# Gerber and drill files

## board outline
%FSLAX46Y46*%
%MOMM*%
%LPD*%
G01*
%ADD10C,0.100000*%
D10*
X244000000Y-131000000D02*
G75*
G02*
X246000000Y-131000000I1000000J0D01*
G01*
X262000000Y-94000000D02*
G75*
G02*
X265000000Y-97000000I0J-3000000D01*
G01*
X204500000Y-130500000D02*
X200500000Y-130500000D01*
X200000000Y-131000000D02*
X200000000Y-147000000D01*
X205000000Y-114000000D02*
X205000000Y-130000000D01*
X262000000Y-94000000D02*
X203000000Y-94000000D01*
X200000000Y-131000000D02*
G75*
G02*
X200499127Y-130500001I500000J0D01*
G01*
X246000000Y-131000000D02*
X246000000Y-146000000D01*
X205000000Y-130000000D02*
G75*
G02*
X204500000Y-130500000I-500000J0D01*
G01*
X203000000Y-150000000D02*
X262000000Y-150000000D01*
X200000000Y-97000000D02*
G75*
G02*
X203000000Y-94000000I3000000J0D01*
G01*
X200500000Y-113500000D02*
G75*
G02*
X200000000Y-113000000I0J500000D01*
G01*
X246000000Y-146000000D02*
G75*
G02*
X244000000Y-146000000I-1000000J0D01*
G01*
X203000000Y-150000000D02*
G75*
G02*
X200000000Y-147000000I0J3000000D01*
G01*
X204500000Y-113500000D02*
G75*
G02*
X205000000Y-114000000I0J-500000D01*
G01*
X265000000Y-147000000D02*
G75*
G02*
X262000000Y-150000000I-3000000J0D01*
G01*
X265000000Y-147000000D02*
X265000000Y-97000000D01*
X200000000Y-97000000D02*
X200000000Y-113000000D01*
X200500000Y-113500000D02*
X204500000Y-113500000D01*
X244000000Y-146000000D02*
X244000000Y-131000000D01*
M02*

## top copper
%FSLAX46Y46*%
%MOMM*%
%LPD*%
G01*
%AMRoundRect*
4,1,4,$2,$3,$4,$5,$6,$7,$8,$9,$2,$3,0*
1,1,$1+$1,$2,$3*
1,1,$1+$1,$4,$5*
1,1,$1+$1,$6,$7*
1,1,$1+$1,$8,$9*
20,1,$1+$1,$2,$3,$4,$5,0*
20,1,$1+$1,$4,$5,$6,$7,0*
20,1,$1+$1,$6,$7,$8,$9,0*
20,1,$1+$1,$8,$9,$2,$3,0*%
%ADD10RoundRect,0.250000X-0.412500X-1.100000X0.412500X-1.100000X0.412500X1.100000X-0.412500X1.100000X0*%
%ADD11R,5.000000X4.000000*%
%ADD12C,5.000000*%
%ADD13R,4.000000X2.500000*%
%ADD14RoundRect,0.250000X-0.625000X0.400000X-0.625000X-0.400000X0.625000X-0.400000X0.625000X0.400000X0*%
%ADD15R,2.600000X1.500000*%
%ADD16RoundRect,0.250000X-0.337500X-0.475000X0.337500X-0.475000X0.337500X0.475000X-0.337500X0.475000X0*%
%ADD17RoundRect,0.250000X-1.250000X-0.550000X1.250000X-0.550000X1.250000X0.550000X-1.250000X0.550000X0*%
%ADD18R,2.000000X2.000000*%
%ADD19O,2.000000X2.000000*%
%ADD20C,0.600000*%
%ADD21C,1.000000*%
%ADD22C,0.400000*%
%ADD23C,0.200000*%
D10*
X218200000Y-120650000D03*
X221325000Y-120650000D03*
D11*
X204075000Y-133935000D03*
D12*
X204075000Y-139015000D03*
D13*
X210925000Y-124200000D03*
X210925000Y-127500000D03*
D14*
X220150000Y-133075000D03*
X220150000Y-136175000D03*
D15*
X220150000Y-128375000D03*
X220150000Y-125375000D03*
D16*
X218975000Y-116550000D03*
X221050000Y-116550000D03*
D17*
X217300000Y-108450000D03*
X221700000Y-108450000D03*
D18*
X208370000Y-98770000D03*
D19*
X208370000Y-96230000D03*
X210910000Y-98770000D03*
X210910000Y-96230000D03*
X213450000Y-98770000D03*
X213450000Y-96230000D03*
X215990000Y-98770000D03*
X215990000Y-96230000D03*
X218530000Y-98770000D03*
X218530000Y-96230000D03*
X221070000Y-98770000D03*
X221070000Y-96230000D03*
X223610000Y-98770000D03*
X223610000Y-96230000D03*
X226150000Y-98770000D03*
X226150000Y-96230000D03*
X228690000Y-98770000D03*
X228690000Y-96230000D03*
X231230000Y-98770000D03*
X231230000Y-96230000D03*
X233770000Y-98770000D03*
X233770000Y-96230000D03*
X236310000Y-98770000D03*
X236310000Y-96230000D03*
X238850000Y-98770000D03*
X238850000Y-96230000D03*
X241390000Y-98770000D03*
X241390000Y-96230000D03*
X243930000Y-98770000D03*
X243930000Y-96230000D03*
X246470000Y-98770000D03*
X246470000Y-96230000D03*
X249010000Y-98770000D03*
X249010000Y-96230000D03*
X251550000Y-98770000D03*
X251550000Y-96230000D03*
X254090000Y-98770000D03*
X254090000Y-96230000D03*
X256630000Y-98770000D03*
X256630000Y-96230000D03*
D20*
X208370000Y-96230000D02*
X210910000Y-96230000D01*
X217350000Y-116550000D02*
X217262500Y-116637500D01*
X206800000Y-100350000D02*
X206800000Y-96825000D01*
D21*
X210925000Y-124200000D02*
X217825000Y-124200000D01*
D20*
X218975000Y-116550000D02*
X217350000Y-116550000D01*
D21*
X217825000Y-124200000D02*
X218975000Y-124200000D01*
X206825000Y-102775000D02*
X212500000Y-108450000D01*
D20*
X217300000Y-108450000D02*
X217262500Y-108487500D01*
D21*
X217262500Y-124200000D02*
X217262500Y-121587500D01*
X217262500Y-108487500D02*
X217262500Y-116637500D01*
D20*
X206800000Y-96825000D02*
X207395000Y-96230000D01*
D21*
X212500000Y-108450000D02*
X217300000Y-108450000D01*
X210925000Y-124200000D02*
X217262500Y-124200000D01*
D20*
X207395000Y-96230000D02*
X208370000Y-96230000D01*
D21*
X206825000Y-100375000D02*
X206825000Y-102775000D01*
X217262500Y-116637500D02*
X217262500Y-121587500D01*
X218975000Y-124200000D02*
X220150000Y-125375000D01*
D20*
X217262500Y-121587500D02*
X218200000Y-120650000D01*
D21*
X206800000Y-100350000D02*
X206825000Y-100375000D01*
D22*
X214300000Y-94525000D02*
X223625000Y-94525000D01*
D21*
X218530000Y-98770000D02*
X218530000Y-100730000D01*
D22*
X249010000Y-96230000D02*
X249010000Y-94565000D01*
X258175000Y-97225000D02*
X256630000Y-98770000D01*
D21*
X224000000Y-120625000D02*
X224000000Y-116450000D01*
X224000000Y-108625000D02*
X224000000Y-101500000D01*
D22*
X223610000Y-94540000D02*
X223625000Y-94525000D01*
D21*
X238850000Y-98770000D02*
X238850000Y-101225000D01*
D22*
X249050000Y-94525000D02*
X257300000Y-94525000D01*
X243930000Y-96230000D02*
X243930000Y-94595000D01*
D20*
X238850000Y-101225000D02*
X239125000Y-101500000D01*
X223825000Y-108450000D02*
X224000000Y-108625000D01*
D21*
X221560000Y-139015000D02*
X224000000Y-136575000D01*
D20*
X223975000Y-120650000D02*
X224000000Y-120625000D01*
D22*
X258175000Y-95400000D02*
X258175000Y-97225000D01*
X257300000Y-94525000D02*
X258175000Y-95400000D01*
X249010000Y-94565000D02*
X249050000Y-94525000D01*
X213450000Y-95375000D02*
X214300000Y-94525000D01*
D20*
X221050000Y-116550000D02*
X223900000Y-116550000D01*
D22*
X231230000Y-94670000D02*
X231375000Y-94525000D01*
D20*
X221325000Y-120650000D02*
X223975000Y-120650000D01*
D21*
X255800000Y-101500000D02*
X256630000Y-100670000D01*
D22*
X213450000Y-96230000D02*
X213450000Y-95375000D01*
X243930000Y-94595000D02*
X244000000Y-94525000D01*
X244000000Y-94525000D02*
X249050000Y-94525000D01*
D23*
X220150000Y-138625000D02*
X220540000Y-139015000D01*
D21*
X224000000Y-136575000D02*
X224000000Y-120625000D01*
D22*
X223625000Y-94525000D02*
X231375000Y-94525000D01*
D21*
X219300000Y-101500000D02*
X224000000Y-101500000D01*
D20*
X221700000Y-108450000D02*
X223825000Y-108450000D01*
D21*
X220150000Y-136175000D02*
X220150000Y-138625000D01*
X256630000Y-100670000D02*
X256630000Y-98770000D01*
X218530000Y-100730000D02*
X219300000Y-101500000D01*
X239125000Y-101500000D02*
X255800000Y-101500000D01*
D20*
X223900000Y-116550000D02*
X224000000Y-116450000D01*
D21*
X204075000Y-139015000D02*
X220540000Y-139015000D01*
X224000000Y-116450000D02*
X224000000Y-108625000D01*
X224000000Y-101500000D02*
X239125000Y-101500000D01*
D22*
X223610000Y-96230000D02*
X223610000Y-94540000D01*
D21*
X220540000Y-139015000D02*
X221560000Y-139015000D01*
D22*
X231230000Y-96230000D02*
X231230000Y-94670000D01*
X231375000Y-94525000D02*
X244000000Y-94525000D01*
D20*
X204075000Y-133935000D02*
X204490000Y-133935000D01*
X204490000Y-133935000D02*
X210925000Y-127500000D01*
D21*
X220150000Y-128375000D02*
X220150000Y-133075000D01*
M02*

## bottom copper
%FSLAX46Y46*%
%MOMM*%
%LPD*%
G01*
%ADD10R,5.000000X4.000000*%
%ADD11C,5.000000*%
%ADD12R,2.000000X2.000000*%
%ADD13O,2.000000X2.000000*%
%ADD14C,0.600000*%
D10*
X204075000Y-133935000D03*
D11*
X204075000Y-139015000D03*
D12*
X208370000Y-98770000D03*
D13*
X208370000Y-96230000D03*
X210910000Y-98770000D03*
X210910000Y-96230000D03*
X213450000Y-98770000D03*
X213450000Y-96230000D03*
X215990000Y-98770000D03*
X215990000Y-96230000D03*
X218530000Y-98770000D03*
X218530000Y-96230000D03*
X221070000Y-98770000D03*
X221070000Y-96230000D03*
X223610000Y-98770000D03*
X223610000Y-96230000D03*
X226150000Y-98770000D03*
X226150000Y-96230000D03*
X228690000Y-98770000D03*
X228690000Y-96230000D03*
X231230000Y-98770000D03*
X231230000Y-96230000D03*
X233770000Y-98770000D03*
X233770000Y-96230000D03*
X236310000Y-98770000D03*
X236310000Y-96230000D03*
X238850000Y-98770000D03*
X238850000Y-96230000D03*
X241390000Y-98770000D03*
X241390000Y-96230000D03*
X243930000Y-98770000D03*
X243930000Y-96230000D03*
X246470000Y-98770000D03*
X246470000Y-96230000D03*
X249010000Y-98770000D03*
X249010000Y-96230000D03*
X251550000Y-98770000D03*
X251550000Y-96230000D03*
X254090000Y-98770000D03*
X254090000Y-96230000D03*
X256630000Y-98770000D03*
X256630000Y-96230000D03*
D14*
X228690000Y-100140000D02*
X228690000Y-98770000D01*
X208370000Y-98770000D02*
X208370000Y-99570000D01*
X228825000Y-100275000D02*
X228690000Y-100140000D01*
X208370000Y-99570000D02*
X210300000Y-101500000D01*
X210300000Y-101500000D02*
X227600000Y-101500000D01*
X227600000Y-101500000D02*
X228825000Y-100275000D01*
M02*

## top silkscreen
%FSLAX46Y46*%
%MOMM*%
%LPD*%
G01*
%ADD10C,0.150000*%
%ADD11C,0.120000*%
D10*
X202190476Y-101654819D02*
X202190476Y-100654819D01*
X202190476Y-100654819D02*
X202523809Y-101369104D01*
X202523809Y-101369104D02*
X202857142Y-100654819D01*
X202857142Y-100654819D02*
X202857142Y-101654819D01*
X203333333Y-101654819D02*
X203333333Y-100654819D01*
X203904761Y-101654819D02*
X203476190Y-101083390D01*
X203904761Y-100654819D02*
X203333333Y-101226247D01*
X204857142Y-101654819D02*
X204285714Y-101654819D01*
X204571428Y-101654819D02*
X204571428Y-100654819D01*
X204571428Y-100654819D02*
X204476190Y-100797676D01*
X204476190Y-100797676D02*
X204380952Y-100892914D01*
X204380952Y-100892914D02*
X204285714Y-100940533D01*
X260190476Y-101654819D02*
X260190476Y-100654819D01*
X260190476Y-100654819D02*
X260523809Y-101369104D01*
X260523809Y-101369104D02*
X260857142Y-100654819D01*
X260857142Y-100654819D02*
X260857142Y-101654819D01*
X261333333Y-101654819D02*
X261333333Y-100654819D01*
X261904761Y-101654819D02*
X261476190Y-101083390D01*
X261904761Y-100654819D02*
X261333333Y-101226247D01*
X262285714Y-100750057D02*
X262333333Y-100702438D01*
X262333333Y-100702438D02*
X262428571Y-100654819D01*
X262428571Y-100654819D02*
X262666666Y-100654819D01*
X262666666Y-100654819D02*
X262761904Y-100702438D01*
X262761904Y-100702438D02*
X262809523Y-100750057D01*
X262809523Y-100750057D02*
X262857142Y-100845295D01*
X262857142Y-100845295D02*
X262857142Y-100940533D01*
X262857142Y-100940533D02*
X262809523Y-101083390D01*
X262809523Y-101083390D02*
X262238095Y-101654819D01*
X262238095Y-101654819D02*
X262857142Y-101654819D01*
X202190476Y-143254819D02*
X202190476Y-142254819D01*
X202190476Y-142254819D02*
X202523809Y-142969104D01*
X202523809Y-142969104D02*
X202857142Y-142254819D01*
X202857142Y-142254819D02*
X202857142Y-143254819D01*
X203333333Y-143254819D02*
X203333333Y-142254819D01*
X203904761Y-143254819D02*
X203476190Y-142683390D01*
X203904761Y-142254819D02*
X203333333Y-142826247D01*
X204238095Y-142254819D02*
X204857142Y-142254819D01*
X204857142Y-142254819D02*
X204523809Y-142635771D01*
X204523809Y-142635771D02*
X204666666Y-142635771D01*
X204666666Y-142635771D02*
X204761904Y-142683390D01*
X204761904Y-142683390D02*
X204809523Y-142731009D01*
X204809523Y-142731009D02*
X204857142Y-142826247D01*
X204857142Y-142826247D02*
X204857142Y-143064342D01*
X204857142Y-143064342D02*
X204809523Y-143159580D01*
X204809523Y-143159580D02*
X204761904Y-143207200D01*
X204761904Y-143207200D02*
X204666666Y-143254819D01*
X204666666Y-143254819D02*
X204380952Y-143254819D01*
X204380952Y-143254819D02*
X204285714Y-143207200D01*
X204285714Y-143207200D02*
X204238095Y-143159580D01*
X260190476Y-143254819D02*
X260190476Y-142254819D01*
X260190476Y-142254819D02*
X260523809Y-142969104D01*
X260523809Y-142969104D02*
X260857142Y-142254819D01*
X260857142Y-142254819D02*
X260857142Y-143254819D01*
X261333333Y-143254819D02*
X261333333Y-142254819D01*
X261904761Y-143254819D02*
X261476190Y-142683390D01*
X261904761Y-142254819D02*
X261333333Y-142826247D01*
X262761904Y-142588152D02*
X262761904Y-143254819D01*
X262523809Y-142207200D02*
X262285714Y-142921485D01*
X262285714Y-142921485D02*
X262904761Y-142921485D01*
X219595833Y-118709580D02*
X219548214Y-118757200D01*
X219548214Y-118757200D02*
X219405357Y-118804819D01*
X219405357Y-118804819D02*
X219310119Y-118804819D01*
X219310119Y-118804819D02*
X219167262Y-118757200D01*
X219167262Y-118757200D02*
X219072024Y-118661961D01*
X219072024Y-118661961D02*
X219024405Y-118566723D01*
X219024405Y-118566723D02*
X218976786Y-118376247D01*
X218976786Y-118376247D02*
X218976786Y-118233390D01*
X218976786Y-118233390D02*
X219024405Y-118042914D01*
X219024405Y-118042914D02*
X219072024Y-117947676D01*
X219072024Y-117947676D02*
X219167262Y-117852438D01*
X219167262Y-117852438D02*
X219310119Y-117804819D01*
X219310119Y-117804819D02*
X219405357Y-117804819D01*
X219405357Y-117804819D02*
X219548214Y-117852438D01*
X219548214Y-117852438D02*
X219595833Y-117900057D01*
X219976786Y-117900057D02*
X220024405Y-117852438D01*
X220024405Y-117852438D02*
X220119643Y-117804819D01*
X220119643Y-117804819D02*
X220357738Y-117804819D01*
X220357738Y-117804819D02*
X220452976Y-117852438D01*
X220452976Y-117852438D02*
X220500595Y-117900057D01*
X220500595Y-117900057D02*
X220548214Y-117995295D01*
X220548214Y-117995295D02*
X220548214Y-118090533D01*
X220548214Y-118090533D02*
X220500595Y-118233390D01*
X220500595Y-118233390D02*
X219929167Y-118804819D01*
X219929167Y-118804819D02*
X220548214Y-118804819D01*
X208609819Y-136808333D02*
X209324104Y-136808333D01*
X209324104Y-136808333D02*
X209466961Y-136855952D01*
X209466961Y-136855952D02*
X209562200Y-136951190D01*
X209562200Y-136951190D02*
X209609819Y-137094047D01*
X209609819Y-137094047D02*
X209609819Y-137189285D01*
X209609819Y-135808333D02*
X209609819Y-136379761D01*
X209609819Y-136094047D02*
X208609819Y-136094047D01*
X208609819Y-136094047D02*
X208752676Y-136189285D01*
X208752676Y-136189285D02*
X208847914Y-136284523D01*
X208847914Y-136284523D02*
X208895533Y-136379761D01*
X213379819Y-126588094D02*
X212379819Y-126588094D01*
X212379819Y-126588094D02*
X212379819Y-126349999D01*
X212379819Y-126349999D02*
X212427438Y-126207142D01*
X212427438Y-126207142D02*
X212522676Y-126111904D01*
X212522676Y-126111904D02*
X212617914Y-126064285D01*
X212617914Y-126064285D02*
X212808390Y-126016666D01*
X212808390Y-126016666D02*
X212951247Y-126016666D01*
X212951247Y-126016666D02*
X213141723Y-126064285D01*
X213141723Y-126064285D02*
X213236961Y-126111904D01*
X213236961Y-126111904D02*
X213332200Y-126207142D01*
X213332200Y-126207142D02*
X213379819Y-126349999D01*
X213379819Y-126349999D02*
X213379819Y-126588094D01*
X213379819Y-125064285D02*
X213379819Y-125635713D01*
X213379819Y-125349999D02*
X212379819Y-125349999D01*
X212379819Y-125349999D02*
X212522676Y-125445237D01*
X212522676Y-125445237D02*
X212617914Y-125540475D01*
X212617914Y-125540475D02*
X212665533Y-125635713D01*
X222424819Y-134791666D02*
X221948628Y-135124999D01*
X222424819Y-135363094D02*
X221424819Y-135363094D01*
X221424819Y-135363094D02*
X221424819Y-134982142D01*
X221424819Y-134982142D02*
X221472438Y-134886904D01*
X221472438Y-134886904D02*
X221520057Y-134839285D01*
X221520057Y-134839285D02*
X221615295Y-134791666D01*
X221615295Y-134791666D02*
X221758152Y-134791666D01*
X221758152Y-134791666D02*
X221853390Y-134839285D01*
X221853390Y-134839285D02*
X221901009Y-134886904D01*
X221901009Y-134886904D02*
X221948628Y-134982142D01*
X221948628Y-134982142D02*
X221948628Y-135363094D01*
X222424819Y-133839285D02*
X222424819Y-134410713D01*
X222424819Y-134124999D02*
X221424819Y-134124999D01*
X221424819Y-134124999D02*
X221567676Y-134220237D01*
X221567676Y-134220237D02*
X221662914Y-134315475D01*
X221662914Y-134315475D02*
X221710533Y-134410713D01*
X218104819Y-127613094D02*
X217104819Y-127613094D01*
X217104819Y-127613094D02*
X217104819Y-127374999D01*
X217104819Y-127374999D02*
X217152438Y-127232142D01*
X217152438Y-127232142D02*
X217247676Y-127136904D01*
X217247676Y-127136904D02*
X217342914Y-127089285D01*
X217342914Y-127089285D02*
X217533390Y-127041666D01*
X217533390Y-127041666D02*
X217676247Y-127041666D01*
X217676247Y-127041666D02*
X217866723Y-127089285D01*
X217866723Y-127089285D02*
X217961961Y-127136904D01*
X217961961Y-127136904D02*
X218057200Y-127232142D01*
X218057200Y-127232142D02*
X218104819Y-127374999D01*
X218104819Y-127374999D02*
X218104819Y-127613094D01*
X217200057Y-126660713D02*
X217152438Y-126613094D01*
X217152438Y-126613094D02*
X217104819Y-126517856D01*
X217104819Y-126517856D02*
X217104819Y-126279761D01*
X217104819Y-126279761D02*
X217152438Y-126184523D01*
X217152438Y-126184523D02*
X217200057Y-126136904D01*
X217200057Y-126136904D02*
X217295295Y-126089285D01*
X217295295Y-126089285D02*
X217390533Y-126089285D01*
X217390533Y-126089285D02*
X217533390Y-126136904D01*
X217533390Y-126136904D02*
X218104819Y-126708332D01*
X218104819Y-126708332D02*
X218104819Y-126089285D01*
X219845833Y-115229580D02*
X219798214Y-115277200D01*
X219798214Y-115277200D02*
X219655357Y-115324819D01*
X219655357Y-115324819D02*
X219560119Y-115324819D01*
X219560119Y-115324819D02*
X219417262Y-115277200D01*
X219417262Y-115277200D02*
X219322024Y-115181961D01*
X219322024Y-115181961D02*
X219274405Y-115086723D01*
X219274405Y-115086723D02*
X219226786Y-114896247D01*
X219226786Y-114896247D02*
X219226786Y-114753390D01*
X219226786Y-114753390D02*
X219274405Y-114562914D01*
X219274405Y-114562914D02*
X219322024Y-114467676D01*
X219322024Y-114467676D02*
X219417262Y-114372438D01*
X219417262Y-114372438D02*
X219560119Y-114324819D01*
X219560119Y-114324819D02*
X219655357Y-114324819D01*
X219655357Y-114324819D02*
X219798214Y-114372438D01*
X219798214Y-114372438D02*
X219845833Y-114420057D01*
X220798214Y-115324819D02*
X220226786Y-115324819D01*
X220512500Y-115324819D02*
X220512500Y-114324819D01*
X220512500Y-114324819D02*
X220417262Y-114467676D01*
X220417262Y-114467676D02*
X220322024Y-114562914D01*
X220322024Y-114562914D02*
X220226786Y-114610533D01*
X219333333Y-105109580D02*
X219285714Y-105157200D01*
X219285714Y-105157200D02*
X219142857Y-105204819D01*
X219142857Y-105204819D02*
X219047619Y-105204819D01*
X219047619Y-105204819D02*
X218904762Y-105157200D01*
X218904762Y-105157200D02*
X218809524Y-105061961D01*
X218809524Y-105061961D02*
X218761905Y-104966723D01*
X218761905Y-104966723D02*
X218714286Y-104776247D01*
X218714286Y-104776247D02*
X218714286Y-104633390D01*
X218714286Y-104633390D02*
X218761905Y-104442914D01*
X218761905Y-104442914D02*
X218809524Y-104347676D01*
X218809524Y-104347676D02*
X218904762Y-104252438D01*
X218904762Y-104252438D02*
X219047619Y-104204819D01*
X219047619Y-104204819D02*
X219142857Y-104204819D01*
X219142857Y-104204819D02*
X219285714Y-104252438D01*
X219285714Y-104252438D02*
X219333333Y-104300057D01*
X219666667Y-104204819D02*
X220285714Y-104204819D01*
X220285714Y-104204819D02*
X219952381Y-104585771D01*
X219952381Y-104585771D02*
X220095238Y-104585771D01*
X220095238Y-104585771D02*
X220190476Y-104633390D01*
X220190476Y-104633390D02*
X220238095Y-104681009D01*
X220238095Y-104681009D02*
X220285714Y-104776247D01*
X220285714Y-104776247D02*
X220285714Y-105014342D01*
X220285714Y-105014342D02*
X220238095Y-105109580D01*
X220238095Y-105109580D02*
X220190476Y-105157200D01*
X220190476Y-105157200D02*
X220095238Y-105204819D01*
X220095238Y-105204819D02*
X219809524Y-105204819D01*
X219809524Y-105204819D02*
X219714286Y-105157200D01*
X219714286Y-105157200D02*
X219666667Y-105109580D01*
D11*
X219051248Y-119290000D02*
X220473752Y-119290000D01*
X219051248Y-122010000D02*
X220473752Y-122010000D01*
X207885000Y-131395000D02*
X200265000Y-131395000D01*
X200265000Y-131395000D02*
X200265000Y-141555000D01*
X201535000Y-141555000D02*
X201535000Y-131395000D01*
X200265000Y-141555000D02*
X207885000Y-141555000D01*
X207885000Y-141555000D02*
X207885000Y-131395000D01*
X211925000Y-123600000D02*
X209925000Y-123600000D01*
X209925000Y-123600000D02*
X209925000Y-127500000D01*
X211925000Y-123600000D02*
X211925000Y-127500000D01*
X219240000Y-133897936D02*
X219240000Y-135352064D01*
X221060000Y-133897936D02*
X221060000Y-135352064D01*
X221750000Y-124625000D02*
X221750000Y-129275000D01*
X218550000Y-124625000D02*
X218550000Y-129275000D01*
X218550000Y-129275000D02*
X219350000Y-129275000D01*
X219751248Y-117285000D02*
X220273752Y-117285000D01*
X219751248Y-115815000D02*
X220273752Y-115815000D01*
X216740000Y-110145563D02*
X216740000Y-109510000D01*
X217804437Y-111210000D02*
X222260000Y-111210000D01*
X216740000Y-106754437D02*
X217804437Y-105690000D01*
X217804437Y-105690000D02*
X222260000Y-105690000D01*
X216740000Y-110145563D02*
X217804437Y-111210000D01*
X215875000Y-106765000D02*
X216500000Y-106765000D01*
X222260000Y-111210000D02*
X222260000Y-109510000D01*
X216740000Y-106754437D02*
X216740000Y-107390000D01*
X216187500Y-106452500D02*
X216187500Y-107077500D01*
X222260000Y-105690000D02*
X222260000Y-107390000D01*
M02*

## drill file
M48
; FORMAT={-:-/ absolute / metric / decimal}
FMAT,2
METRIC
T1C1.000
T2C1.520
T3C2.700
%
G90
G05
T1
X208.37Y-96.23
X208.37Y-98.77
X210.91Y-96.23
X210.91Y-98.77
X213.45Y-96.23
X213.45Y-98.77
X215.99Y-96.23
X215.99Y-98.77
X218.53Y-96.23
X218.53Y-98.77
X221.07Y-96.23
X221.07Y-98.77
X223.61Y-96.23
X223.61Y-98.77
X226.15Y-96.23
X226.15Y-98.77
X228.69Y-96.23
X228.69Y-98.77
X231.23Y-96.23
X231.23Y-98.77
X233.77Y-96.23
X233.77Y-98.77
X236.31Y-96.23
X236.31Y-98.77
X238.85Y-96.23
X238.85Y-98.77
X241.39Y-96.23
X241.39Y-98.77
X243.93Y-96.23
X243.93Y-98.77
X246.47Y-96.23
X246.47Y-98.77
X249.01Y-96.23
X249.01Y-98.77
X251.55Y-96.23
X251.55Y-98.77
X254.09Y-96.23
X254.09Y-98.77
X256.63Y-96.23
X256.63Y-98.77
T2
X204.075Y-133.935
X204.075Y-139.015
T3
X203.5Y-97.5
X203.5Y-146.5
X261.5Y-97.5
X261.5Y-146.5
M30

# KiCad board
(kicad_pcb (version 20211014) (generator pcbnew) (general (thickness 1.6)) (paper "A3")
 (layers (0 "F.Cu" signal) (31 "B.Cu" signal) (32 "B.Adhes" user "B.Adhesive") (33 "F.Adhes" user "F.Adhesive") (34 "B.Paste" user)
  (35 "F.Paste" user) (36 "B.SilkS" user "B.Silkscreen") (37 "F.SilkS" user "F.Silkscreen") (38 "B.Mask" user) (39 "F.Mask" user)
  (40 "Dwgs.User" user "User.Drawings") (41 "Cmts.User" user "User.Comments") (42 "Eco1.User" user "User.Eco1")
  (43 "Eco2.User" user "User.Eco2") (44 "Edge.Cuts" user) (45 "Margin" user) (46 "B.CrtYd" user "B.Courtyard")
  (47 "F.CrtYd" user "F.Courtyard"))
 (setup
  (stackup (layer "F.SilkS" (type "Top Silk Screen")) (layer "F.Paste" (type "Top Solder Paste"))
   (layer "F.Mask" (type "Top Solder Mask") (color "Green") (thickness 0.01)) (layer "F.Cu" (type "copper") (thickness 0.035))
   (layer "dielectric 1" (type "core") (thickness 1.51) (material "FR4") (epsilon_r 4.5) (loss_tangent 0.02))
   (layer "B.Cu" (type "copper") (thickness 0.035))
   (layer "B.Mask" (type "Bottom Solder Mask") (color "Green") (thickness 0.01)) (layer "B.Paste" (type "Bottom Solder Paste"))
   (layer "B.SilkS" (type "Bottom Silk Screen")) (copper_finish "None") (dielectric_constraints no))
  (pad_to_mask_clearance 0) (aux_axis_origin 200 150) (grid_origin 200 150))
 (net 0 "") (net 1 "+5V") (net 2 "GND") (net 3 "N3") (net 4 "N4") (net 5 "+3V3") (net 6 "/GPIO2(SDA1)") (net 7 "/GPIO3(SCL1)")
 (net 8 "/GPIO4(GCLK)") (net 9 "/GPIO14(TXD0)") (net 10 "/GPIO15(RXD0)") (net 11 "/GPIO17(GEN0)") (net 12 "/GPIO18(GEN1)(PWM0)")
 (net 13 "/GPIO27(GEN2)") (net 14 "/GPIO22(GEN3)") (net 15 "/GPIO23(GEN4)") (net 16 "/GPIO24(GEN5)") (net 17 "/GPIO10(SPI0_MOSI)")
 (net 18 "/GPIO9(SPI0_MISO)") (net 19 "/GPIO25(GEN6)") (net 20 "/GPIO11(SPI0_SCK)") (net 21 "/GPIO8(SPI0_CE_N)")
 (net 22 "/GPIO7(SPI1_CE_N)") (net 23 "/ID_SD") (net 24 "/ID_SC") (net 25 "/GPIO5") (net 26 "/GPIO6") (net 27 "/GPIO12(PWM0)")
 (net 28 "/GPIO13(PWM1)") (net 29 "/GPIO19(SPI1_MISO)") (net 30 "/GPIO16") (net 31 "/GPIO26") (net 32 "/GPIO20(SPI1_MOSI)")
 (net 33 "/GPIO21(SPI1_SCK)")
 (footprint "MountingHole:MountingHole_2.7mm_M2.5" (layer "F.Cu") (at 203.5 97.5 180)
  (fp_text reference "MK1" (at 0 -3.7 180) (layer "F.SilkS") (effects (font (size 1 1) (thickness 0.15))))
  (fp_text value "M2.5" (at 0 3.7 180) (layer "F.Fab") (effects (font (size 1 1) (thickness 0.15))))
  (pad "" np_thru_hole circle locked (at 0 0 180) (size 2.7 2.7) (drill 2.7) (layers *.Cu *.Mask)))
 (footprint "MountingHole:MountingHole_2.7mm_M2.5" (layer "F.Cu") (at 261.5 97.5 180)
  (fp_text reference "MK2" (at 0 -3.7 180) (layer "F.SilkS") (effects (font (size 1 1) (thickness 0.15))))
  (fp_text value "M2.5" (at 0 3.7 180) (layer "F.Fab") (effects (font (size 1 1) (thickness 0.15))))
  (pad "" np_thru_hole circle locked (at 0 0 180) (size 2.7 2.7) (drill 2.7) (layers *.Cu *.Mask)))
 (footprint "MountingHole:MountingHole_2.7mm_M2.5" (layer "F.Cu") (at 203.5 146.5)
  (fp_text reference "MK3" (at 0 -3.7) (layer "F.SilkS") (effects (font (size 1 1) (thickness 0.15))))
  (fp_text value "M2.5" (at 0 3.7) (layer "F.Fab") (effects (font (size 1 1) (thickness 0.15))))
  (pad "" np_thru_hole circle locked (at 0 0) (size 2.7 2.7) (drill 2.7) (layers *.Cu *.Mask)))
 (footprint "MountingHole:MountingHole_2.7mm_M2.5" (layer "F.Cu") (at 261.5 146.5)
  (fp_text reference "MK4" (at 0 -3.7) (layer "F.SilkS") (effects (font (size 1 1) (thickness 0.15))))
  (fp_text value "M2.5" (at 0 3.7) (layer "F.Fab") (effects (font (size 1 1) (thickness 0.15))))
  (pad "" np_thru_hole circle locked (at 0 0) (size 2.7 2.7) (drill 2.7) (layers *.Cu *.Mask)))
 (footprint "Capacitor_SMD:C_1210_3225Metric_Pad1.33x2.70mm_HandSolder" (layer "F.Cu") (at 219.7625 120.65)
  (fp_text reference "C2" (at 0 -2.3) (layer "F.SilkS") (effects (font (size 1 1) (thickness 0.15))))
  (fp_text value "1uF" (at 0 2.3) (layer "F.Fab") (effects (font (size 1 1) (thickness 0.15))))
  (fp_line (start -0.711252 -1.36) (end 0.711252 -1.36) (layer "F.SilkS") (width 0.12))
  (fp_line (start -0.711252 1.36) (end 0.711252 1.36) (layer "F.SilkS") (width 0.12))
  (pad "1" smd roundrect locked (at -1.5625 0) (size 1.325 2.7) (layers "F.Cu" "F.Paste" "F.Mask") (roundrect_rratio 0.1886792453)
   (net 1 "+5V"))
  (pad "2" smd roundrect locked (at 1.5625 0) (size 1.325 2.7) (layers "F.Cu" "F.Paste" "F.Mask") (roundrect_rratio 0.1886792453)
   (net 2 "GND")))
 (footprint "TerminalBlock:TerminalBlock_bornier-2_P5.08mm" (layer "F.Cu") (at 204.075 133.935 -90)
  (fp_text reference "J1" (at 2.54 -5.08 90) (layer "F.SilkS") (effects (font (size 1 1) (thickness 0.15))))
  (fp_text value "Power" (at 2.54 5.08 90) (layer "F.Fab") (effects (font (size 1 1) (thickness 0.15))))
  (fp_line (start -2.54 -3.81) (end -2.54 3.81) (layer "F.SilkS") (width 0.12))
  (fp_line (start -2.54 3.81) (end 7.62 3.81) (layer "F.SilkS") (width 0.12))
  (fp_line (start 7.62 2.54) (end -2.54 2.54) (layer "F.SilkS") (width 0.12))
  (fp_line (start 7.62 3.81) (end 7.62 -3.81) (layer "F.SilkS") (width 0.12))
  (fp_line (start 7.62 -3.81) (end -2.54 -3.81) (layer "F.SilkS") (width 0.12))
  (pad "1" thru_hole rect locked (at 0 0 270) (size 4 5) (drill 1.52) (layers *.Cu *.Mask) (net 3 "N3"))
  (pad "2" thru_hole circle locked (at 5.08 0 270) (size 5 5) (drill 1.52) (layers *.Cu *.Mask) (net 2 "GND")))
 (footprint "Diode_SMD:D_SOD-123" (layer "F.Cu") (at 210.925 125.85 -90)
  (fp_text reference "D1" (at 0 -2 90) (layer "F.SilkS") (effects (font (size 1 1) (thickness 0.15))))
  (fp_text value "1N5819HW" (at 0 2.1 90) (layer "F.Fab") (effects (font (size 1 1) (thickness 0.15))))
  (fp_line (start -2.25 -1) (end -2.25 1) (layer "F.SilkS") (width 0.12))
  (fp_line (start -2.25 1) (end 1.65 1) (layer "F.SilkS") (width 0.12))
  (fp_line (start -2.25 -1) (end 1.65 -1) (layer "F.SilkS") (width 0.12))
  (pad "1" smd rect locked (at -1.65 0 270) (size 2.5 4) (layers "F.Cu" "F.Paste" "F.Mask") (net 1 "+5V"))
  (pad "2" smd rect locked (at 1.65 0 270) (size 2.5 4) (layers "F.Cu" "F.Paste" "F.Mask") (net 3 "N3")))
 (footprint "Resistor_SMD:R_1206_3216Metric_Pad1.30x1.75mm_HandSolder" (layer "F.Cu") (at 220.15 134.625 -90)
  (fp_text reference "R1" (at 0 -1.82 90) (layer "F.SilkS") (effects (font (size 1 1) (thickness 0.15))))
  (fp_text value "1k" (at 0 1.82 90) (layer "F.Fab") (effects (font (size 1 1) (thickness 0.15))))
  (fp_line (start -0.727064 0.91) (end 0.727064 0.91) (layer "F.SilkS") (width 0.12))
  (fp_line (start -0.727064 -0.91) (end 0.727064 -0.91) (layer "F.SilkS") (width 0.12))
  (pad "1" smd roundrect locked (at -1.55 0 270) (size 1.3 1.75) (layers "F.Cu" "F.Paste" "F.Mask") (roundrect_rratio 0.1923076923)
   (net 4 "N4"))
  (pad "2" smd roundrect locked (at 1.55 0 270) (size 1.3 1.75) (layers "F.Cu" "F.Paste" "F.Mask") (roundrect_rratio 0.1923076923)
   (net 2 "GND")))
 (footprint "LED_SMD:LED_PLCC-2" (layer "F.Cu") (at 220.15 126.875 90)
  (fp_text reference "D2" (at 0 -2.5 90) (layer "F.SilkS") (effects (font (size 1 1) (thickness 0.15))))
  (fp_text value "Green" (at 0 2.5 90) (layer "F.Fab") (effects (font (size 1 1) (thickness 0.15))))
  (fp_line (start 2.25 1.6) (end -2.4 1.6) (layer "F.SilkS") (width 0.12))
  (fp_line (start 2.25 -1.6) (end -2.4 -1.6) (layer "F.SilkS") (width 0.12))
  (fp_line (start -2.4 -1.6) (end -2.4 -0.8) (layer "F.SilkS") (width 0.12))
  (pad "1" smd rect locked (at -1.5 0 90) (size 1.5 2.6) (layers "F.Cu" "F.Paste" "F.Mask") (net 4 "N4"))
  (pad "2" smd rect locked (at 1.5 0 90) (size 1.5 2.6) (layers "F.Cu" "F.Paste" "F.Mask") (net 1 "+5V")))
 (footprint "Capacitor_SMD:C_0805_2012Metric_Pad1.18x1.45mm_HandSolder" (layer "F.Cu") (at 220.0125 116.55)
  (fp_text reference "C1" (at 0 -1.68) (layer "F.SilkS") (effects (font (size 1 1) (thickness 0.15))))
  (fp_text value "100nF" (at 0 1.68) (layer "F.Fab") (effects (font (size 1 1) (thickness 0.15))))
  (fp_line (start -0.261252 0.735) (end 0.261252 0.735) (layer "F.SilkS") (width 0.12))
  (fp_line (start -0.261252 -0.735) (end 0.261252 -0.735) (layer "F.SilkS") (width 0.12))
  (pad "1" smd roundrect locked (at -1.0375 0) (size 1.175 1.45) (layers "F.Cu" "F.Paste" "F.Mask") (roundrect_rratio 0.2127659574)
   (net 1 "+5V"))
  (pad "2" smd roundrect locked (at 1.0375 0) (size 1.175 1.45) (layers "F.Cu" "F.Paste" "F.Mask") (roundrect_rratio 0.2127659574)
   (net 2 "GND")))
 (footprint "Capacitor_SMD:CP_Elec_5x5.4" (layer "F.Cu") (at 219.5 108.45)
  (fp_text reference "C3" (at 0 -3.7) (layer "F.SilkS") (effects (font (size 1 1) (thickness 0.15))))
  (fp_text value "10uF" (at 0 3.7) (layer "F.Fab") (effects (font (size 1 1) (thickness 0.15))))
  (fp_line (start -2.76 1.695563) (end -2.76 1.06) (layer "F.SilkS") (width 0.12))
  (fp_line (start -1.695563 2.76) (end 2.76 2.76) (layer "F.SilkS") (width 0.12))
  (fp_line (start -2.76 -1.695563) (end -1.695563 -2.76) (layer "F.SilkS") (width 0.12))
  (fp_line (start -1.695563 -2.76) (end 2.76 -2.76) (layer "F.SilkS") (width 0.12))
  (fp_line (start -2.76 1.695563) (end -1.695563 2.76) (layer "F.SilkS") (width 0.12))
  (fp_line (start -3.625 -1.685) (end -3 -1.685) (layer "F.SilkS") (width 0.12))
  (fp_line (start 2.76 2.76) (end 2.76 1.06) (layer "F.SilkS") (width 0.12))
  (fp_line (start -2.76 -1.695563) (end -2.76 -1.06) (layer "F.SilkS") (width 0.12))
  (fp_line (start -3.3125 -1.9975) (end -3.3125 -1.3725) (layer "F.SilkS") (width 0.12))
  (fp_line (start 2.76 -2.76) (end 2.76 -1.06) (layer "F.SilkS") (width 0.12))
  (pad "1" smd roundrect locked (at -2.2 0) (size 3 1.6) (layers "F.Cu" "F.Paste" "F.Mask") (roundrect_rratio 0.15625) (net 1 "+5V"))
  (pad "2" smd roundrect locked (at 2.2 0) (size 3 1.6) (layers "F.Cu" "F.Paste" "F.Mask") (roundrect_rratio 0.15625) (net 2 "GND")))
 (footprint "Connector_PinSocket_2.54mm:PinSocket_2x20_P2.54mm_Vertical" (layer "B.Cu") (at 208.37 98.77 -90)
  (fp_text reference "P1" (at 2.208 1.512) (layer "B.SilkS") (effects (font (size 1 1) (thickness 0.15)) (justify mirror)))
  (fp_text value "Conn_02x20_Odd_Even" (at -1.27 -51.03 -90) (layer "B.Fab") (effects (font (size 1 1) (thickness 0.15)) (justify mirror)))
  (pad "1" thru_hole rect locked (at 0 0 270) (size 2 2) (drill 1) (layers *.Cu *.Mask) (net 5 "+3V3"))
  (pad "2" thru_hole oval locked (at -2.54 0 270) (size 2 2) (drill 1) (layers *.Cu *.Mask) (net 1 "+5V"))
  (pad "3" thru_hole oval locked (at 0 -2.54 270) (size 2 2) (drill 1) (layers *.Cu *.Mask) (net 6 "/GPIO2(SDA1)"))
  (pad "4" thru_hole oval locked (at -2.54 -2.54 270) (size 2 2) (drill 1) (layers *.Cu *.Mask) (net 1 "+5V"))
  (pad "5" thru_hole oval locked (at 0 -5.08 270) (size 2 2) (drill 1) (layers *.Cu *.Mask) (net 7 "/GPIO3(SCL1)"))
  (pad "6" thru_hole oval locked (at -2.54 -5.08 270) (size 2 2) (drill 1) (layers *.Cu *.Mask) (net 2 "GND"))
  (pad "7" thru_hole oval locked (at 0 -7.62 270) (size 2 2) (drill 1) (layers *.Cu *.Mask) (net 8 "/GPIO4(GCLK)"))
  (pad "8" thru_hole oval locked (at -2.54 -7.62 270) (size 2 2) (drill 1) (layers *.Cu *.Mask) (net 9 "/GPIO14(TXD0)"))
  (pad "9" thru_hole oval locked (at 0 -10.16 270) (size 2 2) (drill 1) (layers *.Cu *.Mask) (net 2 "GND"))
  (pad "10" thru_hole oval locked (at -2.54 -10.16 270) (size 2 2) (drill 1) (layers *.Cu *.Mask) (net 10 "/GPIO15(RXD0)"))
  (pad "11" thru_hole oval locked (at 0 -12.7 270) (size 2 2) (drill 1) (layers *.Cu *.Mask) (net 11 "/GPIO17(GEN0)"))
  (pad "12" thru_hole oval locked (at -2.54 -12.7 270) (size 2 2) (drill 1) (layers *.Cu *.Mask) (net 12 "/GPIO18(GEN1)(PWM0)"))
  (pad "13" thru_hole oval locked (at 0 -15.24 270) (size 2 2) (drill 1) (layers *.Cu *.Mask) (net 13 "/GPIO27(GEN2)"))
  (pad "14" thru_hole oval locked (at -2.54 -15.24 270) (size 2 2) (drill 1) (layers *.Cu *.Mask) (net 2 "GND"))
  (pad "15" thru_hole oval locked (at 0 -17.78 270) (size 2 2) (drill 1) (layers *.Cu *.Mask) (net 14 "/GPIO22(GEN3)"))
  (pad "16" thru_hole oval locked (at -2.54 -17.78 270) (size 2 2) (drill 1) (layers *.Cu *.Mask) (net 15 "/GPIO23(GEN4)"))
  (pad "17" thru_hole oval locked (at 0 -20.32 270) (size 2 2) (drill 1) (layers *.Cu *.Mask) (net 5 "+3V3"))
  (pad "18" thru_hole oval locked (at -2.54 -20.32 270) (size 2 2) (drill 1) (layers *.Cu *.Mask) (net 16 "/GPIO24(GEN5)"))
  (pad "19" thru_hole oval locked (at 0 -22.86 270) (size 2 2) (drill 1) (layers *.Cu *.Mask) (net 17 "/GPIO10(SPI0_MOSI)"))
  (pad "20" thru_hole oval locked (at -2.54 -22.86 270) (size 2 2) (drill 1) (layers *.Cu *.Mask) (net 2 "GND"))
  (pad "21" thru_hole oval locked (at 0 -25.4 270) (size 2 2) (drill 1) (layers *.Cu *.Mask) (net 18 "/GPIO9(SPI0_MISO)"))
  (pad "22" thru_hole oval locked (at -2.54 -25.4 270) (size 2 2) (drill 1) (layers *.Cu *.Mask) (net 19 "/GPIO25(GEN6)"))
  (pad "23" thru_hole oval locked (at 0 -27.94 270) (size 2 2) (drill 1) (layers *.Cu *.Mask) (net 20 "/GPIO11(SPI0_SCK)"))
  (pad "24" thru_hole oval locked (at -2.54 -27.94 270) (size 2 2) (drill 1) (layers *.Cu *.Mask) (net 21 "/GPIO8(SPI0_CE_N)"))
  (pad "25" thru_hole oval locked (at 0 -30.48 270) (size 2 2) (drill 1) (layers *.Cu *.Mask) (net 2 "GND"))
  (pad "26" thru_hole oval locked (at -2.54 -30.48 270) (size 2 2) (drill 1) (layers *.Cu *.Mask) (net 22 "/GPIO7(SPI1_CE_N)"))
  (pad "27" thru_hole oval locked (at 0 -33.02 270) (size 2 2) (drill 1) (layers *.Cu *.Mask) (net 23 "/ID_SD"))
  (pad "28" thru_hole oval locked (at -2.54 -33.02 270) (size 2 2) (drill 1) (layers *.Cu *.Mask) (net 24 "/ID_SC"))
  (pad "29" thru_hole oval locked (at 0 -35.56 270) (size 2 2) (drill 1) (layers *.Cu *.Mask) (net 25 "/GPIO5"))
  (pad "30" thru_hole oval locked (at -2.54 -35.56 270) (size 2 2) (drill 1) (layers *.Cu *.Mask) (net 2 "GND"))
  (pad "31" thru_hole oval locked (at 0 -38.1 270) (size 2 2) (drill 1) (layers *.Cu *.Mask) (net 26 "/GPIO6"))
  (pad "32" thru_hole oval locked (at -2.54 -38.1 270) (size 2 2) (drill 1) (layers *.Cu *.Mask) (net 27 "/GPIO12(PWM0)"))
  (pad "33" thru_hole oval locked (at 0 -40.64 270) (size 2 2) (drill 1) (layers *.Cu *.Mask) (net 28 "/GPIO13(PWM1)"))
  (pad "34" thru_hole oval locked (at -2.54 -40.64 270) (size 2 2) (drill 1) (layers *.Cu *.Mask) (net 2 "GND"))
  (pad "35" thru_hole oval locked (at 0 -43.18 270) (size 2 2) (drill 1) (layers *.Cu *.Mask) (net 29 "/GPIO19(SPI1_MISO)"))
  (pad "36" thru_hole oval locked (at -2.54 -43.18 270) (size 2 2) (drill 1) (layers *.Cu *.Mask) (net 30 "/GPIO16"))
  (pad "37" thru_hole oval locked (at 0 -45.72 270) (size 2 2) (drill 1) (layers *.Cu *.Mask) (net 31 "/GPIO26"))
  (pad "38" thru_hole oval locked (at -2.54 -45.72 270) (size 2 2) (drill 1) (layers *.Cu *.Mask) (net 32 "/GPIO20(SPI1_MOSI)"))
  (pad "39" thru_hole oval locked (at 0 -48.26 270) (size 2 2) (drill 1) (layers *.Cu *.Mask) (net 2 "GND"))
  (pad "40" thru_hole oval locked (at -2.54 -48.26 270) (size 2 2) (drill 1) (layers *.Cu *.Mask) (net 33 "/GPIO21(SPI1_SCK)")))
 (gr_arc (start 244 131) (mid 245 130) (end 246 131) (layer "Edge.Cuts") (width 0.1))
 (gr_arc (start 262 94) (mid 264.12132 94.87868) (end 265 97) (layer "Edge.Cuts") (width 0.1))
 (gr_line (start 204.5 130.5) (end 200.5 130.5) (layer "Edge.Cuts") (width 0.1))
 (gr_line (start 200 131) (end 200 147) (layer "Edge.Cuts") (width 0.1))
 (gr_line (start 205 114) (end 205 130) (layer "Edge.Cuts") (width 0.1))
 (gr_line (start 262 94) (end 203 94) (layer "Edge.Cuts") (width 0.1))
 (gr_arc (start 200 131) (mid 200.146138 130.646755) (end 200.499127 130.500001) (layer "Edge.Cuts") (width 0.1))
 (gr_line (start 246 131) (end 246 146) (layer "Edge.Cuts") (width 0.1))
 (gr_arc (start 205 130) (mid 204.853553 130.353553) (end 204.5 130.5) (layer "Edge.Cuts") (width 0.1))
 (gr_line (start 203 150) (end 262 150) (layer "Edge.Cuts") (width 0.1))
 (gr_arc (start 200 97) (mid 200.87868 94.87868) (end 203 94) (layer "Edge.Cuts") (width 0.1))
 (gr_arc (start 200.5 113.5) (mid 200.146447 113.353553) (end 200 113) (layer "Edge.Cuts") (width 0.1))
 (gr_arc (start 246 146) (mid 245 147) (end 244 146) (layer "Edge.Cuts") (width 0.1))
 (gr_arc (start 203 150) (mid 200.87868 149.12132) (end 200 147) (layer "Edge.Cuts") (width 0.1))
 (gr_arc (start 204.5 113.5) (mid 204.853553 113.646447) (end 205 114) (layer "Edge.Cuts") (width 0.1))
 (gr_arc (start 265 147) (mid 264.12132 149.12132) (end 262 150) (layer "Edge.Cuts") (width 0.1))
 (gr_line (start 265 147) (end 265 97) (layer "Edge.Cuts") (width 0.1))
 (gr_line (start 200 97) (end 200 113) (layer "Edge.Cuts") (width 0.1))
 (gr_line (start 200.5 113.5) (end 204.5 113.5) (layer "Edge.Cuts") (width 0.1))
 (gr_line (start 244 146) (end 244 131) (layer "Edge.Cuts") (width 0.1))
 (segment (start 228.69 100.14) (end 228.69 98.77) (width 0.6) (layer "B.Cu") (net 5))
 (segment (start 208.37 98.77) (end 208.37 99.57) (width 0.6) (layer "B.Cu") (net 5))
 (segment (start 228.825 100.275) (end 228.69 100.14) (width 0.6) (layer "B.Cu") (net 5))
 (segment (start 208.37 99.57) (end 210.3 101.5) (width 0.6) (layer "B.Cu") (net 5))
 (segment (start 210.3 101.5) (end 227.6 101.5) (width 0.6) (layer "B.Cu") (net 5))
 (segment (start 227.6 101.5) (end 228.825 100.275) (width 0.6) (layer "B.Cu") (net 5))
 (segment (start 208.37 96.23) (end 210.91 96.23) (width 0.6) (layer "F.Cu") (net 1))
 (segment (start 217.35 116.55) (end 217.2625 116.6375) (width 0.6) (layer "F.Cu") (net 1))
 (segment (start 206.8 100.35) (end 206.8 96.825) (width 0.6) (layer "F.Cu") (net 1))
 (segment (start 210.925 124.2) (end 217.825 124.2) (width 1) (layer "F.Cu") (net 1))
 (segment (start 218.975 116.55) (end 217.35 116.55) (width 0.6) (layer "F.Cu") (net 1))
 (segment (start 217.825 124.2) (end 218.975 124.2) (width 1) (layer "F.Cu") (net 1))
 (segment (start 206.825 102.775) (end 212.5 108.45) (width 1) (layer "F.Cu") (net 1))
 (segment (start 217.3 108.45) (end 217.2625 108.4875) (width 0.6) (layer "F.Cu") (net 1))
 (segment (start 217.2625 124.2) (end 217.2625 121.5875) (width 1) (layer "F.Cu") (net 1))
 (segment (start 217.2625 108.4875) (end 217.2625 116.6375) (width 1) (layer "F.Cu") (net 1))
 (segment (start 206.8 96.825) (end 207.395 96.23) (width 0.6) (layer "F.Cu") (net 1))
 (segment (start 212.5 108.45) (end 217.3 108.45) (width 1) (layer "F.Cu") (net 1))
 (segment (start 210.925 124.2) (end 217.2625 124.2) (width 1) (layer "F.Cu") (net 1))
 (segment (start 207.395 96.23) (end 208.37 96.23) (width 0.6) (layer "F.Cu") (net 1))
 (segment (start 206.825 100.375) (end 206.825 102.775) (width 1) (layer "F.Cu") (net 1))
 (segment (start 217.2625 116.6375) (end 217.2625 121.5875) (width 1) (layer "F.Cu") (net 1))
 (segment (start 218.975 124.2) (end 220.15 125.375) (width 1) (layer "F.Cu") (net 1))
 (segment (start 217.2625 121.5875) (end 218.2 120.65) (width 0.6) (layer "F.Cu") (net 1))
 (segment (start 206.8 100.35) (end 206.825 100.375) (width 1) (layer "F.Cu") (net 1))
 (segment (start 214.3 94.525) (end 223.625 94.525) (width 0.4) (layer "F.Cu") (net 2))
 (segment (start 218.53 98.77) (end 218.53 100.73) (width 1) (layer "F.Cu") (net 2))
 (segment (start 249.01 96.23) (end 249.01 94.565) (width 0.4) (layer "F.Cu") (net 2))
 (segment (start 258.175 97.225) (end 256.63 98.77) (width 0.4) (layer "F.Cu") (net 2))
 (segment (start 224 120.625) (end 224 116.45) (width 1) (layer "F.Cu") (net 2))
 (segment (start 224 108.625) (end 224 101.5) (width 1) (layer "F.Cu") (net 2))
 (segment (start 223.61 94.54) (end 223.625 94.525) (width 0.4) (layer "F.Cu") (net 2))
 (segment (start 238.85 98.77) (end 238.85 101.225) (width 1) (layer "F.Cu") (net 2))
 (segment (start 249.05 94.525) (end 257.3 94.525) (width 0.4) (layer "F.Cu") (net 2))
 (segment (start 243.93 96.23) (end 243.93 94.595) (width 0.4) (layer "F.Cu") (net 2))
 (segment (start 238.85 101.225) (end 239.125 101.5) (width 0.6) (layer "F.Cu") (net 2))
 (segment (start 223.825 108.45) (end 224 108.625) (width 0.6) (layer "F.Cu") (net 2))
 (segment (start 221.56 139.015) (end 224 136.575) (width 1) (layer "F.Cu") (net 2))
 (segment (start 223.975 120.65) (end 224 120.625) (width 0.6) (layer "F.Cu") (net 2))
 (segment (start 258.175 95.4) (end 258.175 97.225) (width 0.4) (layer "F.Cu") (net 2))
 (segment (start 257.3 94.525) (end 258.175 95.4) (width 0.4) (layer "F.Cu") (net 2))
 (segment (start 249.01 94.565) (end 249.05 94.525) (width 0.4) (layer "F.Cu") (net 2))
 (segment (start 213.45 95.375) (end 214.3 94.525) (width 0.4) (layer "F.Cu") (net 2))
 (segment (start 221.05 116.55) (end 223.9 116.55) (width 0.6) (layer "F.Cu") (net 2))
 (segment (start 231.23 94.67) (end 231.375 94.525) (width 0.4) (layer "F.Cu") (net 2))
 (segment (start 221.325 120.65) (end 223.975 120.65) (width 0.6) (layer "F.Cu") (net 2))
 (segment (start 255.8 101.5) (end 256.63 100.67) (width 1) (layer "F.Cu") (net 2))
 (segment (start 213.45 96.23) (end 213.45 95.375) (width 0.4) (layer "F.Cu") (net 2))
 (segment (start 243.93 94.595) (end 244 94.525) (width 0.4) (layer "F.Cu") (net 2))
 (segment (start 244 94.525) (end 249.05 94.525) (width 0.4) (layer "F.Cu") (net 2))
 (segment (start 220.15 138.625) (end 220.54 139.015) (width 0.2) (layer "F.Cu") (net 2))
 (segment (start 224 136.575) (end 224 120.625) (width 1) (layer "F.Cu") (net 2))
 (segment (start 223.625 94.525) (end 231.375 94.525) (width 0.4) (layer "F.Cu") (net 2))
 (segment (start 219.3 101.5) (end 224 101.5) (width 1) (layer "F.Cu") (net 2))
 (segment (start 221.7 108.45) (end 223.825 108.45) (width 0.6) (layer "F.Cu") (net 2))
 (segment (start 220.15 136.175) (end 220.15 138.625) (width 1) (layer "F.Cu") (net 2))
 (segment (start 256.63 100.67) (end 256.63 98.77) (width 1) (layer "F.Cu") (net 2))
 (segment (start 218.53 100.73) (end 219.3 101.5) (width 1) (layer "F.Cu") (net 2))
 (segment (start 239.125 101.5) (end 255.8 101.5) (width 1) (layer "F.Cu") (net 2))
 (segment (start 223.9 116.55) (end 224 116.45) (width 0.6) (layer "F.Cu") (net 2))
 (segment (start 204.075 139.015) (end 220.54 139.015) (width 1) (layer "F.Cu") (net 2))
 (segment (start 224 116.45) (end 224 108.625) (width 1) (layer "F.Cu") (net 2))
 (segment (start 224 101.5) (end 239.125 101.5) (width 1) (layer "F.Cu") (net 2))
 (segment (start 223.61 96.23) (end 223.61 94.54) (width 0.4) (layer "F.Cu") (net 2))
 (segment (start 220.54 139.015) (end 221.56 139.015) (width 1) (layer "F.Cu") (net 2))
 (segment (start 231.23 96.23) (end 231.23 94.67) (width 0.4) (layer "F.Cu") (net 2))
 (segment (start 231.375 94.525) (end 244 94.525) (width 0.4) (layer "F.Cu") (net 2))
 (segment (start 204.075 133.935) (end 204.49 133.935) (width 0.6) (layer "F.Cu") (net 3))
 (segment (start 204.49 133.935) (end 210.925 127.5) (width 0.6) (layer "F.Cu") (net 3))
 (segment (start 220.15 128.375) (end 220.15 133.075) (width 1) (layer "F.Cu") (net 4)))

